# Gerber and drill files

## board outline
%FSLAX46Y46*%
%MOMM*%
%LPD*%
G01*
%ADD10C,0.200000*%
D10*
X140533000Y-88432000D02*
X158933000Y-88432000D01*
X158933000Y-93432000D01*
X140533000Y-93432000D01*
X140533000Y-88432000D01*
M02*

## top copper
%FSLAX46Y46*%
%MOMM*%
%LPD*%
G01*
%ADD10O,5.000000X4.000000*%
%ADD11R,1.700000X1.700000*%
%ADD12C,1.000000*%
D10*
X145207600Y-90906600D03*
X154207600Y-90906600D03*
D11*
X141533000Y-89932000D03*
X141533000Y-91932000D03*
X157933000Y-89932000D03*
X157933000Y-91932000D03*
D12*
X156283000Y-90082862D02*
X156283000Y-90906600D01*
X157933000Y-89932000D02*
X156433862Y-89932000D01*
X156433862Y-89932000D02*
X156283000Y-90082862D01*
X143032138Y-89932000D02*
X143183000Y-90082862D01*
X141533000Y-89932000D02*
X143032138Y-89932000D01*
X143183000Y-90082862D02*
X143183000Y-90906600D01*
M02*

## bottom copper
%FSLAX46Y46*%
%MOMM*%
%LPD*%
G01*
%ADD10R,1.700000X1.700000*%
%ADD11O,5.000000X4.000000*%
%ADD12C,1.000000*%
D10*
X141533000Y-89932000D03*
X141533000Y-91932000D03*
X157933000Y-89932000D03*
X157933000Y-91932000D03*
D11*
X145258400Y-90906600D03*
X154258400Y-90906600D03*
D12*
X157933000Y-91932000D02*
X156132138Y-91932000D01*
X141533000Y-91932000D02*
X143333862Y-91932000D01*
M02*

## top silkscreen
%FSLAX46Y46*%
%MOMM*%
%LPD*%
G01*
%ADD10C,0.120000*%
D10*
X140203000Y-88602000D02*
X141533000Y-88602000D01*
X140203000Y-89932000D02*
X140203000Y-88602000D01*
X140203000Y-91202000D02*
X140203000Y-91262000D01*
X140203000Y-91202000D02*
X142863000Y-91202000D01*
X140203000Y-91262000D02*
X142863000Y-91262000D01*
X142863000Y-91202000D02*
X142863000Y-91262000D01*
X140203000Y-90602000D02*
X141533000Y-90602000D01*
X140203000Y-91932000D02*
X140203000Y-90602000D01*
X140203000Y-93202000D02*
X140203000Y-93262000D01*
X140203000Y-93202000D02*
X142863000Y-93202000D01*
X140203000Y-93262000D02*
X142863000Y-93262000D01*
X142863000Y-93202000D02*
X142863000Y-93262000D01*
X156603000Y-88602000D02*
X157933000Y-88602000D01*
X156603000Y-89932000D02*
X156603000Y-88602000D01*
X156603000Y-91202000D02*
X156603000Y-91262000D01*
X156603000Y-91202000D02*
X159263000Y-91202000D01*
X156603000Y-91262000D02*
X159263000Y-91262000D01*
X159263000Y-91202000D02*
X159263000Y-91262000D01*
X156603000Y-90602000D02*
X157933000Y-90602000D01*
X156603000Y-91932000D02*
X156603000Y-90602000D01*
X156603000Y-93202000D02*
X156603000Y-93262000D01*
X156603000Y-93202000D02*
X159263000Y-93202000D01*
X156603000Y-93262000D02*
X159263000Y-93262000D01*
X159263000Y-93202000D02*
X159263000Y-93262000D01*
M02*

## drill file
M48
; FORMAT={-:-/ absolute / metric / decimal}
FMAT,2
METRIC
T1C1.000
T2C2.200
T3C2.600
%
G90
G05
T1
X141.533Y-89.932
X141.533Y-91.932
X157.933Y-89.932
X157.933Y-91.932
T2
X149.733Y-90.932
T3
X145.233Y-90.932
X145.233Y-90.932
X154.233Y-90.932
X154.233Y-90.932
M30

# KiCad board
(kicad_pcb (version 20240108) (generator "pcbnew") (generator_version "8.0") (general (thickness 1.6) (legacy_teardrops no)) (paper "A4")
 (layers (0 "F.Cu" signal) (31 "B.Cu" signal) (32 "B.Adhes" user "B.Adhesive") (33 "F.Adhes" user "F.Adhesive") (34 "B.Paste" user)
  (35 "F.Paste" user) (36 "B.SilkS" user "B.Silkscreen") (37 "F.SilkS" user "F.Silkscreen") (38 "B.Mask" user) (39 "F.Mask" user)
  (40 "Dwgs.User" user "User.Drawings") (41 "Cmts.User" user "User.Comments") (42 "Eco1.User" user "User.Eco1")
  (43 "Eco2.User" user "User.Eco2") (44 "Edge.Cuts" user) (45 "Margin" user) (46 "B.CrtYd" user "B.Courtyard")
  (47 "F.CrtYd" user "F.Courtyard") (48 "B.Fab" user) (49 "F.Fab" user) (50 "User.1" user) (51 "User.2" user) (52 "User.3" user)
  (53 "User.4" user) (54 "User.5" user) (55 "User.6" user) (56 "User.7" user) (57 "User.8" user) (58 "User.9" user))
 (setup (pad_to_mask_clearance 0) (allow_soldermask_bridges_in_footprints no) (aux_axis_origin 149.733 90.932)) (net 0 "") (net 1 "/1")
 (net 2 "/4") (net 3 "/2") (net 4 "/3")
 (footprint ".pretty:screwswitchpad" (layer "F.Cu") (at 145.233 90.932)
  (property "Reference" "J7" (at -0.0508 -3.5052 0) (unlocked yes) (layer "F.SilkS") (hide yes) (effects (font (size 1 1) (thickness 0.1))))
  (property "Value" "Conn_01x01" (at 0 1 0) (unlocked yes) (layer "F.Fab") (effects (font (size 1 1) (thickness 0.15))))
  (pad "" np_thru_hole oval (at 0 0) (size 1 1) (drill 2.6) (layers "F&B.Cu" "*.Mask") (clearance 0.01))
  (pad "1" smd oval (at -0.0254 -0.0254) (size 5 4) (layers "F.Cu" "F.Paste" "F.Mask") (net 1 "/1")))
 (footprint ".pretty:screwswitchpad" (layer "F.Cu") (at 154.233 90.932)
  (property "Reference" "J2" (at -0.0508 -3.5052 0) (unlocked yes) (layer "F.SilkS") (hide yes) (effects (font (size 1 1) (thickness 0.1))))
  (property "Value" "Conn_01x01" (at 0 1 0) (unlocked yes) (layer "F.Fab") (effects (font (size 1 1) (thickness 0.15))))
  (pad "" np_thru_hole oval (at 0 0) (size 1 1) (drill 2.6) (layers "F&B.Cu" "*.Mask") (clearance 0.01))
  (pad "1" smd oval (at -0.0254 -0.0254) (size 5 4) (layers "F.Cu" "F.Paste" "F.Mask") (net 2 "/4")))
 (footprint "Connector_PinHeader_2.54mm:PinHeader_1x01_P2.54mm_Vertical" (layer "F.Cu") (at 141.533 89.932)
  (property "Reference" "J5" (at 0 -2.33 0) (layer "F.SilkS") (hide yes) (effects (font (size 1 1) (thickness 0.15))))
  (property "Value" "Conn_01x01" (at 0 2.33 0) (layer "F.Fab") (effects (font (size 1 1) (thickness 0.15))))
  (fp_line (start -1.33 -1.33) (end 0 -1.33) (stroke (width 0.12) (type solid)) (layer "F.SilkS"))
  (fp_line (start -1.33 0) (end -1.33 -1.33) (stroke (width 0.12) (type solid)) (layer "F.SilkS"))
  (fp_line (start -1.33 1.27) (end -1.33 1.33) (stroke (width 0.12) (type solid)) (layer "F.SilkS"))
  (fp_line (start -1.33 1.27) (end 1.33 1.27) (stroke (width 0.12) (type solid)) (layer "F.SilkS"))
  (fp_line (start -1.33 1.33) (end 1.33 1.33) (stroke (width 0.12) (type solid)) (layer "F.SilkS"))
  (fp_line (start 1.33 1.27) (end 1.33 1.33) (stroke (width 0.12) (type solid)) (layer "F.SilkS"))
  (pad "1" thru_hole rect (at 0 0) (size 1.7 1.7) (drill 1) (layers "*.Cu" "*.Mask") (remove_unused_layers no) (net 1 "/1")))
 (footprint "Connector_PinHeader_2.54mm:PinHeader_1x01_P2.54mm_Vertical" (layer "F.Cu") (at 141.533 91.932)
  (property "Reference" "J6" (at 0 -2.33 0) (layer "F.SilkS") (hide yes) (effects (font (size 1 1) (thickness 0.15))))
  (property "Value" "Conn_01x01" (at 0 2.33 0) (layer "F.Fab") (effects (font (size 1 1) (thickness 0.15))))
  (fp_line (start -1.33 -1.33) (end 0 -1.33) (stroke (width 0.12) (type solid)) (layer "F.SilkS"))
  (fp_line (start -1.33 0) (end -1.33 -1.33) (stroke (width 0.12) (type solid)) (layer "F.SilkS"))
  (fp_line (start -1.33 1.27) (end -1.33 1.33) (stroke (width 0.12) (type solid)) (layer "F.SilkS"))
  (fp_line (start -1.33 1.27) (end 1.33 1.27) (stroke (width 0.12) (type solid)) (layer "F.SilkS"))
  (fp_line (start -1.33 1.33) (end 1.33 1.33) (stroke (width 0.12) (type solid)) (layer "F.SilkS"))
  (fp_line (start 1.33 1.27) (end 1.33 1.33) (stroke (width 0.12) (type solid)) (layer "F.SilkS"))
  (pad "1" thru_hole rect (at 0 0) (size 1.7 1.7) (drill 1) (layers "*.Cu" "*.Mask") (remove_unused_layers no) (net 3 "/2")))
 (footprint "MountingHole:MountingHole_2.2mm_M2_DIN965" (layer "F.Cu") (at 149.733 90.932)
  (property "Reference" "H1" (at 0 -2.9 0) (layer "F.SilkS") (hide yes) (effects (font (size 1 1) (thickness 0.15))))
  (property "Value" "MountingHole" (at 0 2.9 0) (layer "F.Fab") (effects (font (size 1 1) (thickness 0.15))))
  (pad "" np_thru_hole circle (at 0 0) (size 2.2 2.2) (drill 2.2) (layers "*.Cu" "*.Mask")))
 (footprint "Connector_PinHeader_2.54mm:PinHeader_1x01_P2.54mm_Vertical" (layer "F.Cu") (at 157.933 89.932)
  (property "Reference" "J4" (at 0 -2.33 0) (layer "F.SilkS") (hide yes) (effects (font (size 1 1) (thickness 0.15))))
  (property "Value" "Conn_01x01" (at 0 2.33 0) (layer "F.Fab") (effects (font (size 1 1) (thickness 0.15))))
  (fp_line (start -1.33 -1.33) (end 0 -1.33) (stroke (width 0.12) (type solid)) (layer "F.SilkS"))
  (fp_line (start -1.33 0) (end -1.33 -1.33) (stroke (width 0.12) (type solid)) (layer "F.SilkS"))
  (fp_line (start -1.33 1.27) (end -1.33 1.33) (stroke (width 0.12) (type solid)) (layer "F.SilkS"))
  (fp_line (start -1.33 1.27) (end 1.33 1.27) (stroke (width 0.12) (type solid)) (layer "F.SilkS"))
  (fp_line (start -1.33 1.33) (end 1.33 1.33) (stroke (width 0.12) (type solid)) (layer "F.SilkS"))
  (fp_line (start 1.33 1.27) (end 1.33 1.33) (stroke (width 0.12) (type solid)) (layer "F.SilkS"))
  (pad "1" thru_hole rect (at 0 0) (size 1.7 1.7) (drill 1) (layers "*.Cu" "*.Mask") (remove_unused_layers no) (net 2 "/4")))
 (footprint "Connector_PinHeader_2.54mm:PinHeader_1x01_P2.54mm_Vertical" (layer "F.Cu") (at 157.933 91.932)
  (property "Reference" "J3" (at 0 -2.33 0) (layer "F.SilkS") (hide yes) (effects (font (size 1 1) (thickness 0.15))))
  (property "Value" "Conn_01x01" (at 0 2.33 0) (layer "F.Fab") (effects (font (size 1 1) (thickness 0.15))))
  (fp_line (start -1.33 -1.33) (end 0 -1.33) (stroke (width 0.12) (type solid)) (layer "F.SilkS"))
  (fp_line (start -1.33 0) (end -1.33 -1.33) (stroke (width 0.12) (type solid)) (layer "F.SilkS"))
  (fp_line (start -1.33 1.27) (end -1.33 1.33) (stroke (width 0.12) (type solid)) (layer "F.SilkS"))
  (fp_line (start -1.33 1.27) (end 1.33 1.27) (stroke (width 0.12) (type solid)) (layer "F.SilkS"))
  (fp_line (start -1.33 1.33) (end 1.33 1.33) (stroke (width 0.12) (type solid)) (layer "F.SilkS"))
  (fp_line (start 1.33 1.27) (end 1.33 1.33) (stroke (width 0.12) (type solid)) (layer "F.SilkS"))
  (pad "1" thru_hole rect (at 0 0) (size 1.7 1.7) (drill 1) (layers "*.Cu" "*.Mask") (remove_unused_layers no) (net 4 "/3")))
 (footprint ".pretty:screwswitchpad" (layer "B.Cu") (at 145.233 90.932 180)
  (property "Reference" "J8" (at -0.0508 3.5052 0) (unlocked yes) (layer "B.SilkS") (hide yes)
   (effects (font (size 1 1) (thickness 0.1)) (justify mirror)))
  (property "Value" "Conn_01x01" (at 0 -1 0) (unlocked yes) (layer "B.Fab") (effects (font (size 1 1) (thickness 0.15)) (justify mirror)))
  (pad "" np_thru_hole oval (at 0 0 180) (size 1 1) (drill 2.6) (layers "F&B.Cu" "*.Mask") (clearance 0.01))
  (pad "1" smd oval (at -0.0254 0.0254 180) (size 5 4) (layers "B.Cu" "B.Paste" "B.Mask") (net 3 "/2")))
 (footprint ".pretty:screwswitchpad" (layer "B.Cu") (at 154.233 90.932 180)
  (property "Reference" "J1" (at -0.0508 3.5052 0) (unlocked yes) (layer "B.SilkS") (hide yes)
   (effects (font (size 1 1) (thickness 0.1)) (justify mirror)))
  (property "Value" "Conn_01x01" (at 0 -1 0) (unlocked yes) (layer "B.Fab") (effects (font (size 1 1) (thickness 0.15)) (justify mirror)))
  (pad "" np_thru_hole oval (at 0 0 180) (size 1 1) (drill 2.6) (layers "F&B.Cu" "*.Mask") (clearance 0.01))
  (pad "1" smd oval (at -0.0254 0.0254 180) (size 5 4) (layers "B.Cu" "B.Paste" "B.Mask") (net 4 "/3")))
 (gr_rect (start 140.533 88.432) (end 158.933 93.432) (stroke (width 0.2) (type default)) (fill none) (layer "Edge.Cuts"))
 (segment (start 157.933 91.932) (end 156.132138 91.932) (width 1) (layer "B.Cu") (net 4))
 (segment (start 156.283 90.082862) (end 156.283 90.9066) (width 1) (layer "F.Cu") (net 2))
 (segment (start 157.933 89.932) (end 156.433862 89.932) (width 1) (layer "F.Cu") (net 2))
 (segment (start 156.433862 89.932) (end 156.283 90.082862) (width 1) (layer "F.Cu") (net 2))
 (segment (start 143.032138 89.932) (end 143.183 90.082862) (width 1) (layer "F.Cu") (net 1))
 (segment (start 141.533 89.932) (end 143.032138 89.932) (width 1) (layer "F.Cu") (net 1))
 (segment (start 143.183 90.082862) (end 143.183 90.9066) (width 1) (layer "F.Cu") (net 1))
 (segment (start 141.533 91.932) (end 143.333862 91.932) (width 1) (layer "B.Cu") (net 3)))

